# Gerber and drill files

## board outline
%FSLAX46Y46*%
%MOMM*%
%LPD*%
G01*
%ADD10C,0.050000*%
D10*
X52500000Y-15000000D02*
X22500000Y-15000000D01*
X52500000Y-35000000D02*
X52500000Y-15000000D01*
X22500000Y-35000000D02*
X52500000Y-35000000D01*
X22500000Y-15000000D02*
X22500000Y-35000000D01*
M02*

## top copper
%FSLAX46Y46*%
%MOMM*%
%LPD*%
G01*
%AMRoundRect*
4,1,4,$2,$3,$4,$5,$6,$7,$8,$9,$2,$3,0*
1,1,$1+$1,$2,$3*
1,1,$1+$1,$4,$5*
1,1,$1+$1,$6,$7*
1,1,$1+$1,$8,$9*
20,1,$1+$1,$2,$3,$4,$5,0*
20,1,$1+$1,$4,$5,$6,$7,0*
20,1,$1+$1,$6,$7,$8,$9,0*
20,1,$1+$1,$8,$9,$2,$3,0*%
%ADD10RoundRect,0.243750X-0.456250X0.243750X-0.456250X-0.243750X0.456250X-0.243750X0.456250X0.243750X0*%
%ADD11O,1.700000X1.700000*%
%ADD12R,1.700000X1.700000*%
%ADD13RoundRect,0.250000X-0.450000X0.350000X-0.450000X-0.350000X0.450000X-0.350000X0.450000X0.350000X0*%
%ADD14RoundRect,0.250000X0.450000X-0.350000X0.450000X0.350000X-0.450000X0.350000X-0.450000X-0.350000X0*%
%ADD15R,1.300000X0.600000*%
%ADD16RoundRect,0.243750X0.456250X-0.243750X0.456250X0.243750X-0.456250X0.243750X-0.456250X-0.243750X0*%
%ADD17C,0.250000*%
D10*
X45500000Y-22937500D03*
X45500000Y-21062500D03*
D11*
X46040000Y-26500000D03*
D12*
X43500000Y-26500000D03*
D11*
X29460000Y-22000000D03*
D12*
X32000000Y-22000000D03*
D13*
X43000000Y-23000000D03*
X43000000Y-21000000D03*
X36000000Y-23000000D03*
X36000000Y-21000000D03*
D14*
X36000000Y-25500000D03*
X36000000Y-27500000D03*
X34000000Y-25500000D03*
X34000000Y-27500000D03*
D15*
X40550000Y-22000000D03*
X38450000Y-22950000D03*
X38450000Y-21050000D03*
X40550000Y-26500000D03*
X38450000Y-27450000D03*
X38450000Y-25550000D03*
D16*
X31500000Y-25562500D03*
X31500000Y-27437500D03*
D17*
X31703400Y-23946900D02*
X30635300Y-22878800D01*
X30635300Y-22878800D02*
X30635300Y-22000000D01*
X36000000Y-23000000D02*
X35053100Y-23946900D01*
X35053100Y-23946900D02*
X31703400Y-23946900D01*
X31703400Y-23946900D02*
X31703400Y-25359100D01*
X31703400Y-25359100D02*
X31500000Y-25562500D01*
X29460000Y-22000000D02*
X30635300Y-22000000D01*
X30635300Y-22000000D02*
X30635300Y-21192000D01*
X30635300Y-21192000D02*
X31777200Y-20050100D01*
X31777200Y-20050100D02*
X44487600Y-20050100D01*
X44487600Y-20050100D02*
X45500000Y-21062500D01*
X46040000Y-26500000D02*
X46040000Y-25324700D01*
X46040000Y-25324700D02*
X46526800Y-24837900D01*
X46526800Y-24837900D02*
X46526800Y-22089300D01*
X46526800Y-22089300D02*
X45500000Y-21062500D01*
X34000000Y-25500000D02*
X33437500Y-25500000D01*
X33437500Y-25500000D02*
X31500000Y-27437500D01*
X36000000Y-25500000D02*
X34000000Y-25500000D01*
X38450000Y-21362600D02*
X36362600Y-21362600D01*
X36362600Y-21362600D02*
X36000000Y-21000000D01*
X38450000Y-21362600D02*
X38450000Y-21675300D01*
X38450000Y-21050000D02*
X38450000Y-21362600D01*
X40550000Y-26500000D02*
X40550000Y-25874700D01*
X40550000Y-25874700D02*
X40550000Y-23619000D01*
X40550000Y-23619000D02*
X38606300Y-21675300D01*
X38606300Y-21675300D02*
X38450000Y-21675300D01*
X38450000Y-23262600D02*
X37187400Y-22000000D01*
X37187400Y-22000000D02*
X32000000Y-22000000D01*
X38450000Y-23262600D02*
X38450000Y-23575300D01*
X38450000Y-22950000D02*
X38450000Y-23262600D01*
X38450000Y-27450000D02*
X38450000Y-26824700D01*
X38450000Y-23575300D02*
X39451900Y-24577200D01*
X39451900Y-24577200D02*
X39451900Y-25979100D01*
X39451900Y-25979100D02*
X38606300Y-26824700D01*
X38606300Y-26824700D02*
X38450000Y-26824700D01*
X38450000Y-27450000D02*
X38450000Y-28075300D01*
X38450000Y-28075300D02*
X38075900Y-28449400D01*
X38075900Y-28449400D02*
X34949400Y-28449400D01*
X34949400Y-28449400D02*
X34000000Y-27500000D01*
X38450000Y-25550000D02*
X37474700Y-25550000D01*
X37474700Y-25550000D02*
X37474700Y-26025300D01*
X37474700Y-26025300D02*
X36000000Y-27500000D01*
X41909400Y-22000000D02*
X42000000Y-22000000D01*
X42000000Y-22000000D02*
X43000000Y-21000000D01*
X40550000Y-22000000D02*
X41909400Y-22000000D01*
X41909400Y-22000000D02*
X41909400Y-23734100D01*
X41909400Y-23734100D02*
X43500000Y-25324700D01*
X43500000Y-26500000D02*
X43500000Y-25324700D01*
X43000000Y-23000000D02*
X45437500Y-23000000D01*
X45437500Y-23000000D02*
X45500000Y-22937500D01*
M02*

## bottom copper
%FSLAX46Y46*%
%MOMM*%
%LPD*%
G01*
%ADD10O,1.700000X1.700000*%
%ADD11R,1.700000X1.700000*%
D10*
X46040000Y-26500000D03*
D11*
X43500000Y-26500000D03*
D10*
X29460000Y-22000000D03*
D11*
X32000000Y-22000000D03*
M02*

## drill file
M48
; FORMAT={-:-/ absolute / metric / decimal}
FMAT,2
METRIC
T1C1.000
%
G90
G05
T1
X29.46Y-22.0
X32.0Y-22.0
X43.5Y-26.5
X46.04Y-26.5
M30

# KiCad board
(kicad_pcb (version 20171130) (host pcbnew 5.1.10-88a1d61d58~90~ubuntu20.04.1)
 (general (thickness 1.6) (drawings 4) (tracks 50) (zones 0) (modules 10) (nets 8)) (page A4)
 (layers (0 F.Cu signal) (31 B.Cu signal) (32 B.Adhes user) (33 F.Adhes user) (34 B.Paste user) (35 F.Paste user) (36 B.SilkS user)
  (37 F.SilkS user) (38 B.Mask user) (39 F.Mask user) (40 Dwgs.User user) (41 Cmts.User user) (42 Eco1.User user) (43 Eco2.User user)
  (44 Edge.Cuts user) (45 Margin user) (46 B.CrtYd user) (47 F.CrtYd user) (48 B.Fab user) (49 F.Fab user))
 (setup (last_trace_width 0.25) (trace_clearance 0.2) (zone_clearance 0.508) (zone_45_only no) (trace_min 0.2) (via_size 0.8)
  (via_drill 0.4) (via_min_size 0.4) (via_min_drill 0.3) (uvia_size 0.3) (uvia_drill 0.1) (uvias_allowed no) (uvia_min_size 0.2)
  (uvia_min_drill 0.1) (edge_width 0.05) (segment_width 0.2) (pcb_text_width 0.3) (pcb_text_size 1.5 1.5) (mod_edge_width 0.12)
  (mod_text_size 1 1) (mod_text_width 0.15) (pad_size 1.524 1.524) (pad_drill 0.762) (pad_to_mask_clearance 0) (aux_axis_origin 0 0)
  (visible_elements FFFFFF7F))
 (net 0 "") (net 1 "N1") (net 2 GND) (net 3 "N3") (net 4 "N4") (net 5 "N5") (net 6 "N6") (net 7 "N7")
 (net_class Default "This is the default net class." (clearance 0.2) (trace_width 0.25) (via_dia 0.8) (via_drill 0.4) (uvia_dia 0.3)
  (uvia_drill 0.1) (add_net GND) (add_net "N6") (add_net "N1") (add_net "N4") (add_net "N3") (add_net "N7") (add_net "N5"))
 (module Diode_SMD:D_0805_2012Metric (layer F.Cu) (at 45.5 22 270)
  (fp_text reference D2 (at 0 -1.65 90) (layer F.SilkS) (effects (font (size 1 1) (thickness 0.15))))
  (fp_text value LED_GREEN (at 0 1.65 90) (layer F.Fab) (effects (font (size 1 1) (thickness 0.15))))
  (pad 2 smd roundrect (at 0.9375 0 270) (size 0.975 1.4) (layers F.Cu F.Paste F.Mask) (roundrect_rratio 0.25) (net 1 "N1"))
  (pad 1 smd roundrect (at -0.9375 0 270) (size 0.975 1.4) (layers F.Cu F.Paste F.Mask) (roundrect_rratio 0.25) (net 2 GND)))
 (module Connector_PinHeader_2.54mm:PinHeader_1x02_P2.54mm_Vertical (layer F.Cu) (at 43.5 26.5 90)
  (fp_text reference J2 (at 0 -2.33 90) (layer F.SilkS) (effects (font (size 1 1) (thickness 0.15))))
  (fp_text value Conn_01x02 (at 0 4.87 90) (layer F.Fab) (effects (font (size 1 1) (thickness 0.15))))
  (pad 2 thru_hole oval (at 0 2.54 90) (size 1.7 1.7) (drill 1) (layers *.Cu *.Mask) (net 2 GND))
  (pad 1 thru_hole rect (at 0 0 90) (size 1.7 1.7) (drill 1) (layers *.Cu *.Mask) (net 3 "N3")))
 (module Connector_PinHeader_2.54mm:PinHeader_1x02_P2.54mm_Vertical (layer F.Cu) (at 32 22 270)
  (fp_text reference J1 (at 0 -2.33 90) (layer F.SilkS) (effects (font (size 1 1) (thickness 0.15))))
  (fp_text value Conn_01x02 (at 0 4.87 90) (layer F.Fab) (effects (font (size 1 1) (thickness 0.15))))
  (pad 2 thru_hole oval (at 0 2.54 270) (size 1.7 1.7) (drill 1) (layers *.Cu *.Mask) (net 2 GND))
  (pad 1 thru_hole rect (at 0 0 270) (size 1.7 1.7) (drill 1) (layers *.Cu *.Mask) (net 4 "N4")))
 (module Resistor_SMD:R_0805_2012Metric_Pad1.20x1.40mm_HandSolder (layer F.Cu) (at 43 22 270)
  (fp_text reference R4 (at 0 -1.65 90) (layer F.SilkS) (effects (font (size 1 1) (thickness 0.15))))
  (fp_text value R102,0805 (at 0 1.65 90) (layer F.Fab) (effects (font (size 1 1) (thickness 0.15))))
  (pad 2 smd roundrect (at 1 0 270) (size 1.2 1.4) (layers F.Cu F.Paste F.Mask) (roundrect_rratio 0.208333) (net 1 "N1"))
  (pad 1 smd roundrect (at -1 0 270) (size 1.2 1.4) (layers F.Cu F.Paste F.Mask) (roundrect_rratio 0.208333) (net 3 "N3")))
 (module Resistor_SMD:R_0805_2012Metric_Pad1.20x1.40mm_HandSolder (layer F.Cu) (at 36 22 270)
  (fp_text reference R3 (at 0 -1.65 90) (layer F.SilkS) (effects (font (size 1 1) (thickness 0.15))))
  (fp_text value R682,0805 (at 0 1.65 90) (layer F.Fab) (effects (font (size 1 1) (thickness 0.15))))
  (pad 2 smd roundrect (at 1 0 270) (size 1.2 1.4) (layers F.Cu F.Paste F.Mask) (roundrect_rratio 0.208333) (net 2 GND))
  (pad 1 smd roundrect (at -1 0 270) (size 1.2 1.4) (layers F.Cu F.Paste F.Mask) (roundrect_rratio 0.208333) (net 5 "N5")))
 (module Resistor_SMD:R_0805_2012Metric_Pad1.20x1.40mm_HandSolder (layer F.Cu) (at 36 26.5 90)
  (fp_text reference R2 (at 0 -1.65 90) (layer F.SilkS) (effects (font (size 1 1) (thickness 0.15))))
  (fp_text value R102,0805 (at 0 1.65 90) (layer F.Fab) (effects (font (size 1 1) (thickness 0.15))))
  (pad 2 smd roundrect (at 1 0 90) (size 1.2 1.4) (layers F.Cu F.Paste F.Mask) (roundrect_rratio 0.208333) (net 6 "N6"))
  (pad 1 smd roundrect (at -1 0 90) (size 1.2 1.4) (layers F.Cu F.Paste F.Mask) (roundrect_rratio 0.208333) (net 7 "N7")))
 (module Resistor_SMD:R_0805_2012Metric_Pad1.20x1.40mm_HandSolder (layer F.Cu) (at 34 26.5 90)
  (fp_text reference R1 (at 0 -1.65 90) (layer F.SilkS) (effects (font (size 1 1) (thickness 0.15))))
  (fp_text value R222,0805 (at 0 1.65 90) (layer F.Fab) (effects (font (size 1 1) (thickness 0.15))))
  (pad 2 smd roundrect (at 1 0 90) (size 1.2 1.4) (layers F.Cu F.Paste F.Mask) (roundrect_rratio 0.208333) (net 6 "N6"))
  (pad 1 smd roundrect (at -1 0 90) (size 1.2 1.4) (layers F.Cu F.Paste F.Mask) (roundrect_rratio 0.208333) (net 4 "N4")))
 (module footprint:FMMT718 (layer F.Cu) (at 39.5 22)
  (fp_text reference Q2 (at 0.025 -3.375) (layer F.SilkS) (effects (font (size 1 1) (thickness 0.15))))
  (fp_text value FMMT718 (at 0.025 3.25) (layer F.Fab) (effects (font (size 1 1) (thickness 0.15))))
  (pad 3 smd rect (at 1.05 0) (size 1.3 0.6) (layers F.Cu F.Paste F.Mask) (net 3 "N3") (solder_mask_margin 0.07))
  (pad 2 smd rect (at -1.05 0.95) (size 1.3 0.6) (layers F.Cu F.Paste F.Mask) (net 4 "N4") (solder_mask_margin 0.07))
  (pad 1 smd rect (at -1.05 -0.95) (size 1.3 0.6) (layers F.Cu F.Paste F.Mask) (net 5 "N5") (solder_mask_margin 0.07)))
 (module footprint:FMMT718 (layer F.Cu) (at 39.5 26.5)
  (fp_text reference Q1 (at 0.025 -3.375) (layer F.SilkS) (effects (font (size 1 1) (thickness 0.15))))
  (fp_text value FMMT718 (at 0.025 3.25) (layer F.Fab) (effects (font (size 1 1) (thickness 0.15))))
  (pad 3 smd rect (at 1.05 0) (size 1.3 0.6) (layers F.Cu F.Paste F.Mask) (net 5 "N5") (solder_mask_margin 0.07))
  (pad 2 smd rect (at -1.05 0.95) (size 1.3 0.6) (layers F.Cu F.Paste F.Mask) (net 4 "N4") (solder_mask_margin 0.07))
  (pad 1 smd rect (at -1.05 -0.95) (size 1.3 0.6) (layers F.Cu F.Paste F.Mask) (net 7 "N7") (solder_mask_margin 0.07)))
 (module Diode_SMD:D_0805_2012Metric (layer F.Cu) (at 31.5 26.5 90)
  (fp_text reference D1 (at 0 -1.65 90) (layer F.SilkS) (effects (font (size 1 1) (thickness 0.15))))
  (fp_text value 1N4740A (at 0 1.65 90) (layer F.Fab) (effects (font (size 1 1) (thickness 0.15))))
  (pad 2 smd roundrect (at 0.9375 0 90) (size 0.975 1.4) (layers F.Cu F.Paste F.Mask) (roundrect_rratio 0.25) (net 2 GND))
  (pad 1 smd roundrect (at -0.9375 0 90) (size 0.975 1.4) (layers F.Cu F.Paste F.Mask) (roundrect_rratio 0.25) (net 6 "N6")))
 (gr_line (start 52.5 15) (end 22.5 15) (layer Edge.Cuts) (width 0.05))
 (gr_line (start 52.5 35) (end 52.5 15) (layer Edge.Cuts) (width 0.05))
 (gr_line (start 22.5 35) (end 52.5 35) (layer Edge.Cuts) (width 0.05))
 (gr_line (start 22.5 15) (end 22.5 35) (layer Edge.Cuts) (width 0.05))
 (segment (start 31.7034 23.9469) (end 30.6353 22.8788) (width 0.25) (layer F.Cu) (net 2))
 (segment (start 30.6353 22.8788) (end 30.6353 22) (width 0.25) (layer F.Cu) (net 2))
 (segment (start 36 23) (end 35.0531 23.9469) (width 0.25) (layer F.Cu) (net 2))
 (segment (start 35.0531 23.9469) (end 31.7034 23.9469) (width 0.25) (layer F.Cu) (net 2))
 (segment (start 31.7034 23.9469) (end 31.7034 25.3591) (width 0.25) (layer F.Cu) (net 2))
 (segment (start 31.7034 25.3591) (end 31.5 25.5625) (width 0.25) (layer F.Cu) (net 2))
 (segment (start 29.46 22) (end 30.6353 22) (width 0.25) (layer F.Cu) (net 2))
 (segment (start 30.6353 22) (end 30.6353 21.192) (width 0.25) (layer F.Cu) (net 2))
 (segment (start 30.6353 21.192) (end 31.7772 20.0501) (width 0.25) (layer F.Cu) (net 2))
 (segment (start 31.7772 20.0501) (end 44.4876 20.0501) (width 0.25) (layer F.Cu) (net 2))
 (segment (start 44.4876 20.0501) (end 45.5 21.0625) (width 0.25) (layer F.Cu) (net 2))
 (segment (start 46.04 26.5) (end 46.04 25.3247) (width 0.25) (layer F.Cu) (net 2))
 (segment (start 46.04 25.3247) (end 46.5268 24.8379) (width 0.25) (layer F.Cu) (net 2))
 (segment (start 46.5268 24.8379) (end 46.5268 22.0893) (width 0.25) (layer F.Cu) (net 2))
 (segment (start 46.5268 22.0893) (end 45.5 21.0625) (width 0.25) (layer F.Cu) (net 2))
 (segment (start 34 25.5) (end 33.4375 25.5) (width 0.25) (layer F.Cu) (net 6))
 (segment (start 33.4375 25.5) (end 31.5 27.4375) (width 0.25) (layer F.Cu) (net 6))
 (segment (start 36 25.5) (end 34 25.5) (width 0.25) (layer F.Cu) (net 6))
 (segment (start 38.45 21.3626) (end 36.3626 21.3626) (width 0.25) (layer F.Cu) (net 5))
 (segment (start 36.3626 21.3626) (end 36 21) (width 0.25) (layer F.Cu) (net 5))
 (segment (start 38.45 21.3626) (end 38.45 21.6753) (width 0.25) (layer F.Cu) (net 5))
 (segment (start 38.45 21.05) (end 38.45 21.3626) (width 0.25) (layer F.Cu) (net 5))
 (segment (start 40.55 26.5) (end 40.55 25.8747) (width 0.25) (layer F.Cu) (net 5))
 (segment (start 40.55 25.8747) (end 40.55 23.619) (width 0.25) (layer F.Cu) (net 5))
 (segment (start 40.55 23.619) (end 38.6063 21.6753) (width 0.25) (layer F.Cu) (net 5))
 (segment (start 38.6063 21.6753) (end 38.45 21.6753) (width 0.25) (layer F.Cu) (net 5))
 (segment (start 38.45 23.2626) (end 37.1874 22) (width 0.25) (layer F.Cu) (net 4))
 (segment (start 37.1874 22) (end 32 22) (width 0.25) (layer F.Cu) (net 4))
 (segment (start 38.45 23.2626) (end 38.45 23.5753) (width 0.25) (layer F.Cu) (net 4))
 (segment (start 38.45 22.95) (end 38.45 23.2626) (width 0.25) (layer F.Cu) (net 4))
 (segment (start 38.45 27.45) (end 38.45 26.8247) (width 0.25) (layer F.Cu) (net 4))
 (segment (start 38.45 23.5753) (end 39.4519 24.5772) (width 0.25) (layer F.Cu) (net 4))
 (segment (start 39.4519 24.5772) (end 39.4519 25.9791) (width 0.25) (layer F.Cu) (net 4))
 (segment (start 39.4519 25.9791) (end 38.6063 26.8247) (width 0.25) (layer F.Cu) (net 4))
 (segment (start 38.6063 26.8247) (end 38.45 26.8247) (width 0.25) (layer F.Cu) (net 4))
 (segment (start 38.45 27.45) (end 38.45 28.0753) (width 0.25) (layer F.Cu) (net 4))
 (segment (start 38.45 28.0753) (end 38.0759 28.4494) (width 0.25) (layer F.Cu) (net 4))
 (segment (start 38.0759 28.4494) (end 34.9494 28.4494) (width 0.25) (layer F.Cu) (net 4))
 (segment (start 34.9494 28.4494) (end 34 27.5) (width 0.25) (layer F.Cu) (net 4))
 (segment (start 38.45 25.55) (end 37.4747 25.55) (width 0.25) (layer F.Cu) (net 7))
 (segment (start 37.4747 25.55) (end 37.4747 26.0253) (width 0.25) (layer F.Cu) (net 7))
 (segment (start 37.4747 26.0253) (end 36 27.5) (width 0.25) (layer F.Cu) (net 7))
 (segment (start 41.9094 22) (end 42 22) (width 0.25) (layer F.Cu) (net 3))
 (segment (start 42 22) (end 43 21) (width 0.25) (layer F.Cu) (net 3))
 (segment (start 40.55 22) (end 41.9094 22) (width 0.25) (layer F.Cu) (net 3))
 (segment (start 41.9094 22) (end 41.9094 23.7341) (width 0.25) (layer F.Cu) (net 3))
 (segment (start 41.9094 23.7341) (end 43.5 25.3247) (width 0.25) (layer F.Cu) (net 3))
 (segment (start 43.5 26.5) (end 43.5 25.3247) (width 0.25) (layer F.Cu) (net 3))
 (segment (start 43 23) (end 45.4375 23) (width 0.25) (layer F.Cu) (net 1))
 (segment (start 45.4375 23) (end 45.5 22.9375) (width 0.25) (layer F.Cu) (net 1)))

